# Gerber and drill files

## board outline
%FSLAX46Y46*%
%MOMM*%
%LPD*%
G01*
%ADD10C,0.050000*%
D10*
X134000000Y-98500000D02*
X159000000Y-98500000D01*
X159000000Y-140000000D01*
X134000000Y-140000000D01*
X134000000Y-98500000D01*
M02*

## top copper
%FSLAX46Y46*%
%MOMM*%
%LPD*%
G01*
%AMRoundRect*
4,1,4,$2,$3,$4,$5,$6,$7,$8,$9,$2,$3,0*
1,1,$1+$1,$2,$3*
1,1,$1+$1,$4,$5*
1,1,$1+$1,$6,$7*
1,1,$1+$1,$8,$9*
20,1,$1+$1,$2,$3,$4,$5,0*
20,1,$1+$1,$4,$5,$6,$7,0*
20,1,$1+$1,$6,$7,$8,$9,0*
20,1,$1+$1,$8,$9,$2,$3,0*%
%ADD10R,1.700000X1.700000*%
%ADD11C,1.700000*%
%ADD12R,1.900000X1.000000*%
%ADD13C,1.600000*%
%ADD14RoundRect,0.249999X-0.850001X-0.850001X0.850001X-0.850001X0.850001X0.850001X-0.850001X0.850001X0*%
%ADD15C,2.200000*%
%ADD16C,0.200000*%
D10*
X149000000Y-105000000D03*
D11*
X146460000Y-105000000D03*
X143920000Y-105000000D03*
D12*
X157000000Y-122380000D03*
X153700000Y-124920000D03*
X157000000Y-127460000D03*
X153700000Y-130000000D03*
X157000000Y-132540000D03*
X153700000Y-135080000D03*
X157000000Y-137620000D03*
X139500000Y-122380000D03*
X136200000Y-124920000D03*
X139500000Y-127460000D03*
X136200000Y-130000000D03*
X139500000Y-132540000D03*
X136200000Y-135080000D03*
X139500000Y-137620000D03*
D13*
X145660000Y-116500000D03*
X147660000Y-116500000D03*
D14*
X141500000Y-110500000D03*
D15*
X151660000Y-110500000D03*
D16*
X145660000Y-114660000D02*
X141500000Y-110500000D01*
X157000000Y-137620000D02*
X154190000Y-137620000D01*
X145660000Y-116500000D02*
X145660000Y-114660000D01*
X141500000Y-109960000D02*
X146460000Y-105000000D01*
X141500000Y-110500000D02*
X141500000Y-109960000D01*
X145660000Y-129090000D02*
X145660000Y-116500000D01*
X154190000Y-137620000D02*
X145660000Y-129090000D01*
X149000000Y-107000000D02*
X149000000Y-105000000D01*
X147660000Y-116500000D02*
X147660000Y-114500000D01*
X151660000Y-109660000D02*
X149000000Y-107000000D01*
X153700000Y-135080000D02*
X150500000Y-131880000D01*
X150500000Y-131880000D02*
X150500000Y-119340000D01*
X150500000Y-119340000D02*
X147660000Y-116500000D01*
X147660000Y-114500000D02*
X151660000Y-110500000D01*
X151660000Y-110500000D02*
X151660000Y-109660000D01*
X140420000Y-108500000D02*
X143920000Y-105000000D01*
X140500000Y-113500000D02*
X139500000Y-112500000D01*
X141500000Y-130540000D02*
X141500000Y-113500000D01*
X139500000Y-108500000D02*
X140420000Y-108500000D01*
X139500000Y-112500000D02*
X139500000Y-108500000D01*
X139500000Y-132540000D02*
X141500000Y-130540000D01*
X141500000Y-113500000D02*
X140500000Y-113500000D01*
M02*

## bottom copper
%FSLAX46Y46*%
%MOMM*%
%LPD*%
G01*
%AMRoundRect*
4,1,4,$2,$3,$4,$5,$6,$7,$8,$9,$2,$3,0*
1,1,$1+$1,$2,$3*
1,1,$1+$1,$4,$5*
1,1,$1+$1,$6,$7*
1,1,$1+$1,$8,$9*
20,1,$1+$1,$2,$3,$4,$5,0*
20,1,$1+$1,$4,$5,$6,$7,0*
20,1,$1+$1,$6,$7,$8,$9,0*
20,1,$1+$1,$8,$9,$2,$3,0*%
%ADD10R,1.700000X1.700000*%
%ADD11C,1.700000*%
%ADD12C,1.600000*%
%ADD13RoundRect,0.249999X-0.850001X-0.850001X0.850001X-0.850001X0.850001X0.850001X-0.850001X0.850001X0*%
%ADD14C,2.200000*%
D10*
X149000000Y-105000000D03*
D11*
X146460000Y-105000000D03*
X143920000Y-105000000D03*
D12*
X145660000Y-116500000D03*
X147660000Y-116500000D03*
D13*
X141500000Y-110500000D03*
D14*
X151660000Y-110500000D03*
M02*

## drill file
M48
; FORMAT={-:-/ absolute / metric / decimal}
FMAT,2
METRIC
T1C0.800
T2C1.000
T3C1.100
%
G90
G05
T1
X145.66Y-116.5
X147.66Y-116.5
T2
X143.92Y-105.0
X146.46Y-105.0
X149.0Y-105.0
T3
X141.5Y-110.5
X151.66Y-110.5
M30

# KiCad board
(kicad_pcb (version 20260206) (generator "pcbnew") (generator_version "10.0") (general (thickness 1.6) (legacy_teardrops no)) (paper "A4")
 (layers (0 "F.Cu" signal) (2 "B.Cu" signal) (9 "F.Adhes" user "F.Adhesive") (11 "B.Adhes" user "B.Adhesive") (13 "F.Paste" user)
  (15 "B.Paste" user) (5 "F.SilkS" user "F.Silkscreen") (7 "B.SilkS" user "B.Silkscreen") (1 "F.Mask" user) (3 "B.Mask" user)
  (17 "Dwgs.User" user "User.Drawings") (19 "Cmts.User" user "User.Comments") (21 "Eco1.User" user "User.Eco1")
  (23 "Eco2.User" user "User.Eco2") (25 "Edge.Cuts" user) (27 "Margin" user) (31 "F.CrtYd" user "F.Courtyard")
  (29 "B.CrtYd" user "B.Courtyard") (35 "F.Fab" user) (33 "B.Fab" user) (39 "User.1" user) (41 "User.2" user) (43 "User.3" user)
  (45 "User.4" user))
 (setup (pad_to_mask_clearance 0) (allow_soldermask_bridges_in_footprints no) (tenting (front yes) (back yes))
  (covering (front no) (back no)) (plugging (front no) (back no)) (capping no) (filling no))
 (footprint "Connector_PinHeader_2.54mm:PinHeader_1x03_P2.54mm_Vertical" (layer "F.Cu") (at 149 105 -90)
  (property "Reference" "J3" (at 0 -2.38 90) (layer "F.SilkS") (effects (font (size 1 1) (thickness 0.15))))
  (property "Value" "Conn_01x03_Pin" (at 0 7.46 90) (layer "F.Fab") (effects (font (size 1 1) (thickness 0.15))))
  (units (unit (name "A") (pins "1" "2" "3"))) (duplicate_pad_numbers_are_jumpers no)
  (pad "1" thru_hole rect (at 0 0 270) (size 1.7 1.7) (drill 1) (layers "*.Cu" "*.Mask") (remove_unused_layers no) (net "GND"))
  (pad "2" thru_hole circle (at 0 2.54 270) (size 1.7 1.7) (drill 1) (layers "*.Cu" "*.Mask") (remove_unused_layers no) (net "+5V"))
  (pad "3" thru_hole circle (at 0 5.08 270) (size 1.7 1.7) (drill 1) (layers "*.Cu" "*.Mask") (remove_unused_layers no) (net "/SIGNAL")))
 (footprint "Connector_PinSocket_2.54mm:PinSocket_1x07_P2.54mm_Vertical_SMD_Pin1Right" (layer "F.Cu") (at 155.35 130)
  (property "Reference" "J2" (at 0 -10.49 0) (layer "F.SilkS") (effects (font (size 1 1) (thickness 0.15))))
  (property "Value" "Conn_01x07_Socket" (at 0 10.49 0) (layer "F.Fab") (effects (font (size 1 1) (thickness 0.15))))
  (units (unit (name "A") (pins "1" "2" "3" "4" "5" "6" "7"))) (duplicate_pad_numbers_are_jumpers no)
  (pad "1" smd rect (at 1.65 -7.62) (size 1.9 1) (layers "F.Cu" "F.Mask" "F.Paste") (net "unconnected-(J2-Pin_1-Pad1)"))
  (pad "2" smd rect (at -1.65 -5.08) (size 1.9 1) (layers "F.Cu" "F.Mask" "F.Paste") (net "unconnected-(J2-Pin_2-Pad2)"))
  (pad "3" smd rect (at 1.65 -2.54) (size 1.9 1) (layers "F.Cu" "F.Mask" "F.Paste") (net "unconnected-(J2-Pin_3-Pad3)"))
  (pad "4" smd rect (at -1.65 0) (size 1.9 1) (layers "F.Cu" "F.Mask" "F.Paste") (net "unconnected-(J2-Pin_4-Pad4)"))
  (pad "5" smd rect (at 1.65 2.54) (size 1.9 1) (layers "F.Cu" "F.Mask" "F.Paste") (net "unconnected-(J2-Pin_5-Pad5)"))
  (pad "6" smd rect (at -1.65 5.08) (size 1.9 1) (layers "F.Cu" "F.Mask" "F.Paste") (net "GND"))
  (pad "7" smd rect (at 1.65 7.62) (size 1.9 1) (layers "F.Cu" "F.Mask" "F.Paste") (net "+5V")))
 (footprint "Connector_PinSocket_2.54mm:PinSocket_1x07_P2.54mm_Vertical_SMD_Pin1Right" (layer "F.Cu") (at 137.85 130)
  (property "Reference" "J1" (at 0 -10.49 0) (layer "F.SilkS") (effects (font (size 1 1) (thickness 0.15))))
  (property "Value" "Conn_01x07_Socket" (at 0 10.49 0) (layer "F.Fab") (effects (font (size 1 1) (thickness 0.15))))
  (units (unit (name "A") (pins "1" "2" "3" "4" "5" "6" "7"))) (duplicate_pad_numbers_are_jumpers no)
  (pad "1" smd rect (at 1.65 -7.62) (size 1.9 1) (layers "F.Cu" "F.Mask" "F.Paste") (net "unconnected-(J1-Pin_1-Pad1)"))
  (pad "2" smd rect (at -1.65 -5.08) (size 1.9 1) (layers "F.Cu" "F.Mask" "F.Paste") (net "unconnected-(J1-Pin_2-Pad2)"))
  (pad "3" smd rect (at 1.65 -2.54) (size 1.9 1) (layers "F.Cu" "F.Mask" "F.Paste") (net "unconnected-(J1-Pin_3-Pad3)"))
  (pad "4" smd rect (at -1.65 0) (size 1.9 1) (layers "F.Cu" "F.Mask" "F.Paste") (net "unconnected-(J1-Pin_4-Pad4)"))
  (pad "5" smd rect (at 1.65 2.54) (size 1.9 1) (layers "F.Cu" "F.Mask" "F.Paste") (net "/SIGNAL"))
  (pad "6" smd rect (at -1.65 5.08) (size 1.9 1) (layers "F.Cu" "F.Mask" "F.Paste") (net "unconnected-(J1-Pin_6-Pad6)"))
  (pad "7" smd rect (at 1.65 7.62) (size 1.9 1) (layers "F.Cu" "F.Mask" "F.Paste") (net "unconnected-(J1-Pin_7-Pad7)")))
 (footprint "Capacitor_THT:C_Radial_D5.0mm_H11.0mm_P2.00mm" (layer "F.Cu") (at 145.66 116.5)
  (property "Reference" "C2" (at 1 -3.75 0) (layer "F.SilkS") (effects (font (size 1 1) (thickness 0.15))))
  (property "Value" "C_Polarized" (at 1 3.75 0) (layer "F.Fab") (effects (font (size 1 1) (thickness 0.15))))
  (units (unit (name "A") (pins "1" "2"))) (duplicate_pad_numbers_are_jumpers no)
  (pad "1" thru_hole circle (at 0 0) (size 1.6 1.6) (drill 0.8) (layers "*.Cu" "*.Mask") (remove_unused_layers no) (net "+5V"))
  (pad "2" thru_hole circle (at 2 0) (size 1.6 1.6) (drill 0.8) (layers "*.Cu" "*.Mask") (remove_unused_layers no) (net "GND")))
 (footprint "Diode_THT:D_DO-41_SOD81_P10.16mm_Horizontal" (layer "F.Cu") (at 141.5 110.5)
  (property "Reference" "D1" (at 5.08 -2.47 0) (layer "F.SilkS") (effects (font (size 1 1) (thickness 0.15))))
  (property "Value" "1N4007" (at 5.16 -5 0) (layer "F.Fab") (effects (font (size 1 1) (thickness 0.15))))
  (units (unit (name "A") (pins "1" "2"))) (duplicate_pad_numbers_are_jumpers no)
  (pad "1" thru_hole roundrect (at 0 0) (size 2.2 2.2) (drill 1.1) (layers "*.Cu" "*.Mask") (remove_unused_layers no)
   (roundrect_rratio 0.113636) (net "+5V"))
  (pad "2" thru_hole circle (at 10.16 0) (size 2.2 2.2) (drill 1.1) (layers "*.Cu" "*.Mask") (remove_unused_layers no) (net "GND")))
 (gr_rect (start 134 98.5) (end 159 140) (stroke (width 0.05) (type default)) (fill no) (layer "Edge.Cuts"))
 (segment (start 145.66 114.66) (end 141.5 110.5) (width 0.2) (layer "F.Cu") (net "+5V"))
 (segment (start 157 137.62) (end 154.19 137.62) (width 0.2) (layer "F.Cu") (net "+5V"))
 (segment (start 145.66 116.5) (end 145.66 114.66) (width 0.2) (layer "F.Cu") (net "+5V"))
 (segment (start 141.5 109.96) (end 146.46 105) (width 0.2) (layer "F.Cu") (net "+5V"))
 (segment (start 141.5 110.5) (end 141.5 109.96) (width 0.2) (layer "F.Cu") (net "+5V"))
 (segment (start 145.66 129.09) (end 145.66 116.5) (width 0.2) (layer "F.Cu") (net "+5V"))
 (segment (start 154.19 137.62) (end 145.66 129.09) (width 0.2) (layer "F.Cu") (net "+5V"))
 (segment (start 149 107) (end 149 105) (width 0.2) (layer "F.Cu") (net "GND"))
 (segment (start 147.66 116.5) (end 147.66 114.5) (width 0.2) (layer "F.Cu") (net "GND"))
 (segment (start 151.66 109.66) (end 149 107) (width 0.2) (layer "F.Cu") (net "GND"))
 (segment (start 153.7 135.08) (end 150.5 131.88) (width 0.2) (layer "F.Cu") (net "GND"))
 (segment (start 150.5 131.88) (end 150.5 119.34) (width 0.2) (layer "F.Cu") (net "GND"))
 (segment (start 150.5 119.34) (end 147.66 116.5) (width 0.2) (layer "F.Cu") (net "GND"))
 (segment (start 147.66 114.5) (end 151.66 110.5) (width 0.2) (layer "F.Cu") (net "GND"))
 (segment (start 151.66 110.5) (end 151.66 109.66) (width 0.2) (layer "F.Cu") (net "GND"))
 (segment (start 140.42 108.5) (end 143.92 105) (width 0.2) (layer "F.Cu") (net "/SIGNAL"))
 (segment (start 140.5 113.5) (end 139.5 112.5) (width 0.2) (layer "F.Cu") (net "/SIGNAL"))
 (segment (start 141.5 130.54) (end 141.5 113.5) (width 0.2) (layer "F.Cu") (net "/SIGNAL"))
 (segment (start 139.5 108.5) (end 140.42 108.5) (width 0.2) (layer "F.Cu") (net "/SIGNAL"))
 (segment (start 139.5 112.5) (end 139.5 108.5) (width 0.2) (layer "F.Cu") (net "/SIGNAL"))
 (segment (start 139.5 132.54) (end 141.5 130.54) (width 0.2) (layer "F.Cu") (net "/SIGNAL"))
 (segment (start 141.5 113.5) (end 140.5 113.5) (width 0.2) (layer "F.Cu") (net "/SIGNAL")))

